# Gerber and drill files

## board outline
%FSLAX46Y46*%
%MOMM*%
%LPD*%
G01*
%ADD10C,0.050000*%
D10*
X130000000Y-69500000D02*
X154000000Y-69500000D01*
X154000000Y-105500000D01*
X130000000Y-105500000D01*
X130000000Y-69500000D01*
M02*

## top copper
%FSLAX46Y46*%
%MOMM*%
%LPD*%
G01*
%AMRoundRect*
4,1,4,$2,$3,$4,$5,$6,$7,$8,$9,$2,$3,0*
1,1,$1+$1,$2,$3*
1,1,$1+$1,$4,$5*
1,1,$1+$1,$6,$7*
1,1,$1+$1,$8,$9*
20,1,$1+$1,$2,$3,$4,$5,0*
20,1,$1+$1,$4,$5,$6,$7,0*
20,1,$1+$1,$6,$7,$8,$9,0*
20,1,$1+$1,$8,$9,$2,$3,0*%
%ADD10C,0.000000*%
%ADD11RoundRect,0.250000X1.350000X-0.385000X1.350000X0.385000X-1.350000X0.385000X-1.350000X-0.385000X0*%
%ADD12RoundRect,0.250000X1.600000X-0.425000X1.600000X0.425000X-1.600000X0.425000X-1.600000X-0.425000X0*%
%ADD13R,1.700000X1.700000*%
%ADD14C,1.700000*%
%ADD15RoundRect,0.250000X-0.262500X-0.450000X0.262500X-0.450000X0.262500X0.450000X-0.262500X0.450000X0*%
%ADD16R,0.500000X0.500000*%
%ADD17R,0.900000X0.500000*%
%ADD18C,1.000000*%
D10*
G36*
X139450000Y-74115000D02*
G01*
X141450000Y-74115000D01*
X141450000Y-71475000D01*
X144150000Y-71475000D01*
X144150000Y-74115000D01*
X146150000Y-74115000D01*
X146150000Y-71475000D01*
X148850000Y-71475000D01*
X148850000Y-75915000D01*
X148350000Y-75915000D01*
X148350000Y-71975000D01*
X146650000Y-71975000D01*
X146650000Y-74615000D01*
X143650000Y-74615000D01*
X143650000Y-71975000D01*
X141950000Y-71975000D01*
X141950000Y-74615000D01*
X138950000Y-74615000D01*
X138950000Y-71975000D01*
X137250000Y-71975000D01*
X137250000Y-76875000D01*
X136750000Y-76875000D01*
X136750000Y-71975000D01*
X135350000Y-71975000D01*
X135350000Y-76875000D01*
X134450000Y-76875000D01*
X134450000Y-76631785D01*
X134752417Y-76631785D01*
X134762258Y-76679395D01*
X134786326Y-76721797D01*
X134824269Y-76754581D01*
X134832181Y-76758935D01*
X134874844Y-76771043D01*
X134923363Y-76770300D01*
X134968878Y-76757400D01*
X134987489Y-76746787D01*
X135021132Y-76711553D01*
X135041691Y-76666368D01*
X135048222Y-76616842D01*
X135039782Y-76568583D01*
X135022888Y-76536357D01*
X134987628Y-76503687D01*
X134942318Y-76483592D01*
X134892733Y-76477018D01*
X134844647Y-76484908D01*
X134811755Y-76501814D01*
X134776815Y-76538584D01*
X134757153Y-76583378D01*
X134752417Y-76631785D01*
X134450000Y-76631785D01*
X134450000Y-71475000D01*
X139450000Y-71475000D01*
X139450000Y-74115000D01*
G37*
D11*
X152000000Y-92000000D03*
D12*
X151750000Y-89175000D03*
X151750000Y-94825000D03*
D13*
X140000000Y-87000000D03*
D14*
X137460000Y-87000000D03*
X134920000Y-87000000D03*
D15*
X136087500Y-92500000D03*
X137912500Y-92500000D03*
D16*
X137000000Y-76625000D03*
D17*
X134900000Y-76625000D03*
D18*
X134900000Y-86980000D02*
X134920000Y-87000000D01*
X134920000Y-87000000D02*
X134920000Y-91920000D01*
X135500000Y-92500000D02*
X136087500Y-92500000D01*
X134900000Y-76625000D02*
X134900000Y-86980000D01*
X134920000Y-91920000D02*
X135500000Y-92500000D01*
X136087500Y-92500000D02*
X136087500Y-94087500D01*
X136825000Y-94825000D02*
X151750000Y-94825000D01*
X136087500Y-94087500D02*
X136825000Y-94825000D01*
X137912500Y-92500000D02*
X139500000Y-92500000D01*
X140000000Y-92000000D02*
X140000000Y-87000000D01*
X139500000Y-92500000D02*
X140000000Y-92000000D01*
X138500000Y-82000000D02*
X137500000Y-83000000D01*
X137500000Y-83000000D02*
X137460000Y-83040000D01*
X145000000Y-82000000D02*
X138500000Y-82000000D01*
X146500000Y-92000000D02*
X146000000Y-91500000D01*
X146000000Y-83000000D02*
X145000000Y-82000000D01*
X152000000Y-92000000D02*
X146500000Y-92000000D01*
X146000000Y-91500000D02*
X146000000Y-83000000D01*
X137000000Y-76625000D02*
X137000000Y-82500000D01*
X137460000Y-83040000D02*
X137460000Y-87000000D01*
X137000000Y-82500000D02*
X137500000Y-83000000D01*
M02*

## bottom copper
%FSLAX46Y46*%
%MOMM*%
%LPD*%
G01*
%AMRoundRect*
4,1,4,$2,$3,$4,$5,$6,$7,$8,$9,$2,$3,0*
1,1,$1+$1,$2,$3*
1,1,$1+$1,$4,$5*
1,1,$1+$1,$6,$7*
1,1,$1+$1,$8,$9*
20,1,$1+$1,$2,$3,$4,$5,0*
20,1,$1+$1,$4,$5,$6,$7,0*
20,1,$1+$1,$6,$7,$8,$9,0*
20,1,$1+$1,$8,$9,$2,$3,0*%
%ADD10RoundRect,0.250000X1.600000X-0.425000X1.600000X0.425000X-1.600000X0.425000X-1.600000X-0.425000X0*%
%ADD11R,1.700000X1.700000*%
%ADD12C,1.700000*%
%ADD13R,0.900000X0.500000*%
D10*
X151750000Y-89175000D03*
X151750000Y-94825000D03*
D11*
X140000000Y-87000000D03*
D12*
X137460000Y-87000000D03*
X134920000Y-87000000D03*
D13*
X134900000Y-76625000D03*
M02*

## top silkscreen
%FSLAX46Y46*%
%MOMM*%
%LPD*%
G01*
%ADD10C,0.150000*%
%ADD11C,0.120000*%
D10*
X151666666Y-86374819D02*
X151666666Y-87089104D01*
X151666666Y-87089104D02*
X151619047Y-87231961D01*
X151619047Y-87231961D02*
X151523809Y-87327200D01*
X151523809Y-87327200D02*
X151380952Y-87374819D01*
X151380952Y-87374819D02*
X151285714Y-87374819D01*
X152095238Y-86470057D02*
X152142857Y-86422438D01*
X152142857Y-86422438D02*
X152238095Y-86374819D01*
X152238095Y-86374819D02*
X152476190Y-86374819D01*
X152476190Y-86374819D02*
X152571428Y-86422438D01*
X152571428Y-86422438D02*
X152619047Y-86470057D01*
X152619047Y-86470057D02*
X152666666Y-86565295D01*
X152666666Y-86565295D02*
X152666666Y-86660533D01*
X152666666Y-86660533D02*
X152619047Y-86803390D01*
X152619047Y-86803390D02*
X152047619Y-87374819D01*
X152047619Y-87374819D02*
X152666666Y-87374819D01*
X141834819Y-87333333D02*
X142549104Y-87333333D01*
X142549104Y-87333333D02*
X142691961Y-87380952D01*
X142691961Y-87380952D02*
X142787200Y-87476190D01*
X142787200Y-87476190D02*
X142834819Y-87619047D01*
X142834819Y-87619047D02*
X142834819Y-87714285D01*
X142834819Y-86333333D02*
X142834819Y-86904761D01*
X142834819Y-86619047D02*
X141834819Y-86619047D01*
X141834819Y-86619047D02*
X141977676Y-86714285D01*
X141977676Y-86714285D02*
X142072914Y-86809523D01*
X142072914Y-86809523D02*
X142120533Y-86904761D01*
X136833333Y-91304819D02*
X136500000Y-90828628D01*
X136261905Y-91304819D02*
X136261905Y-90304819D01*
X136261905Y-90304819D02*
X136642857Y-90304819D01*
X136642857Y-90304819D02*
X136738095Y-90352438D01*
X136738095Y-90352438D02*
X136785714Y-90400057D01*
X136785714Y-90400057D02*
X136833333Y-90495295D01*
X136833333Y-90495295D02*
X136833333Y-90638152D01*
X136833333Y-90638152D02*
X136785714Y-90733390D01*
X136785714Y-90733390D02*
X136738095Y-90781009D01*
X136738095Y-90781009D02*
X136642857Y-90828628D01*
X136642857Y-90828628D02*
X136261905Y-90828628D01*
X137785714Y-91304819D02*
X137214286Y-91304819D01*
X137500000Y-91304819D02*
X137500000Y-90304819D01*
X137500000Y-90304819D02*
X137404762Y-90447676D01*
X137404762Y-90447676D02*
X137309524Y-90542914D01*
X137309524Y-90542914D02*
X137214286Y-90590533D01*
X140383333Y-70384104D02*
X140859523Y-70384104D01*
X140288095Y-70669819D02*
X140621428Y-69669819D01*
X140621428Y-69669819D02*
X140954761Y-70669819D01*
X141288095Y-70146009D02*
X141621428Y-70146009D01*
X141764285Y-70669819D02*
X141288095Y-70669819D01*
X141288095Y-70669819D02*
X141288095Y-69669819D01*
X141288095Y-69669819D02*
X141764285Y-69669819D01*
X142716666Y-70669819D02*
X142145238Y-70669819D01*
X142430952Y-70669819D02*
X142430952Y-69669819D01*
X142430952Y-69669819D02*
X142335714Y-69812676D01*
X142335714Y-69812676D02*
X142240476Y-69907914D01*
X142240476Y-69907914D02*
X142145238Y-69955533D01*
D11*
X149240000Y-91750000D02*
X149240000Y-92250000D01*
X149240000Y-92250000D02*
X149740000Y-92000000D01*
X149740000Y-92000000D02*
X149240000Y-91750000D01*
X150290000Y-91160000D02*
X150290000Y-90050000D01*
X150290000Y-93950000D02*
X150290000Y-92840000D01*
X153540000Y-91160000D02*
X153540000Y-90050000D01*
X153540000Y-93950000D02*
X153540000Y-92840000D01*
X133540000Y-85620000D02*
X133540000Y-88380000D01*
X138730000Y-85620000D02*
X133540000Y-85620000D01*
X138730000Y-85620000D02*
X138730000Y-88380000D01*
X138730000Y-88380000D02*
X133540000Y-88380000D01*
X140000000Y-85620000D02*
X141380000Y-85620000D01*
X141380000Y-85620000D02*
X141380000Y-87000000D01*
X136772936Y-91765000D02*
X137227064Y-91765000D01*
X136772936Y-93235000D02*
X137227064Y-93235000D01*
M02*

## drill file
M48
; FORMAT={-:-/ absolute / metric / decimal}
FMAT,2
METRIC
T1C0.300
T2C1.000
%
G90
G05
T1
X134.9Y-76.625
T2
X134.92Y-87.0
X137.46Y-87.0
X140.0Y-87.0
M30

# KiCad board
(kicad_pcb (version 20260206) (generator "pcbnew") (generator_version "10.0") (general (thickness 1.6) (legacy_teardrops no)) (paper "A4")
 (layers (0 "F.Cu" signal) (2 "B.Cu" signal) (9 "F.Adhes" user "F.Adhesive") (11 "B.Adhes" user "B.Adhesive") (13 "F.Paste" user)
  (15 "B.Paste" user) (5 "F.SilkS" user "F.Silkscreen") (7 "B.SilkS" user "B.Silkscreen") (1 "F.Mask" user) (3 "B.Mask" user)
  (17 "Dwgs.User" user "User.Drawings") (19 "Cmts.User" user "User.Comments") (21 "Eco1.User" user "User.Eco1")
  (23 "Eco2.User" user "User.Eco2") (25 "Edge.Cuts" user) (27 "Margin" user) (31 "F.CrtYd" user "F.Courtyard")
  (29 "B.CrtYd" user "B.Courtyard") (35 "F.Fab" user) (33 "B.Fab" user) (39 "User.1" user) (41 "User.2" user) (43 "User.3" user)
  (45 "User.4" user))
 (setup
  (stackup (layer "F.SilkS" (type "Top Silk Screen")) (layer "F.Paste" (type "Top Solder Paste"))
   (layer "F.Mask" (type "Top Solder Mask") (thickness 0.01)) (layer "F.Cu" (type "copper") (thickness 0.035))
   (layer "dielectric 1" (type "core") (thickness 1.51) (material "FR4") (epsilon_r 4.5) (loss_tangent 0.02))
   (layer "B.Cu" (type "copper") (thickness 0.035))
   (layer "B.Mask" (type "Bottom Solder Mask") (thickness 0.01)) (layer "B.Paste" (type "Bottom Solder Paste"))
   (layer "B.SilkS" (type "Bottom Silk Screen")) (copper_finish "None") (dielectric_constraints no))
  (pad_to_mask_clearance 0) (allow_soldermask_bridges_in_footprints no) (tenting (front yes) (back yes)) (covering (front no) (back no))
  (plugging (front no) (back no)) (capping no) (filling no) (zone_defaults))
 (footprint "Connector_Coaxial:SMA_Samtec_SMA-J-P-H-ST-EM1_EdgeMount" (layer "F.Cu") (at 152 92)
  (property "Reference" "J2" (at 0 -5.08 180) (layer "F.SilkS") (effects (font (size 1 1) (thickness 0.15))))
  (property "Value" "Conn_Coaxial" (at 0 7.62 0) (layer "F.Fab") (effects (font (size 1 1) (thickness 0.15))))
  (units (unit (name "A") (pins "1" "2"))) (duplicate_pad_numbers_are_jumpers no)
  (fp_line (start -2.76 -0.25) (end -2.76 0.25) (stroke (width 0.12) (type solid)) (layer "F.SilkS"))
  (fp_line (start -2.76 0.25) (end -2.26 0) (stroke (width 0.12) (type solid)) (layer "F.SilkS"))
  (fp_line (start -2.26 0) (end -2.76 -0.25) (stroke (width 0.12) (type solid)) (layer "F.SilkS"))
  (fp_line (start -1.71 -0.84) (end -1.71 -1.95) (stroke (width 0.12) (type solid)) (layer "F.SilkS"))
  (fp_line (start -1.71 1.95) (end -1.71 0.84) (stroke (width 0.12) (type solid)) (layer "F.SilkS"))
  (fp_line (start 1.54 -0.84) (end 1.54 -1.95) (stroke (width 0.12) (type solid)) (layer "F.SilkS"))
  (fp_line (start 1.54 1.95) (end 1.54 0.84) (stroke (width 0.12) (type solid)) (layer "F.SilkS"))
  (pad "1" smd roundrect (at 0 0 90) (size 1.27 3.2) (layers "F.Cu" "F.Mask") (roundrect_rratio 0.1968503937) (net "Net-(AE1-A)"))
  (pad "2" smd roundrect (at -0.25 -2.825 90) (size 1.35 3.7) (layers "F.Cu" "F.Mask") (roundrect_rratio 0.1851851852) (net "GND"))
  (pad "2" smd roundrect (at -0.25 -2.825 90) (size 1.35 3.7) (layers "B.Cu" "B.Mask") (roundrect_rratio 0.1851851852) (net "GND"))
  (pad "2" smd roundrect (at -0.25 2.825 90) (size 1.35 3.7) (layers "F.Cu" "F.Mask") (roundrect_rratio 0.1851851852) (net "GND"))
  (pad "2" smd roundrect (at -0.25 2.825 90) (size 1.35 3.7) (layers "B.Cu" "B.Mask") (roundrect_rratio 0.1851851852) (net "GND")))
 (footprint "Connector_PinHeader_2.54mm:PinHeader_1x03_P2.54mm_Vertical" (layer "F.Cu") (at 140 87 -90)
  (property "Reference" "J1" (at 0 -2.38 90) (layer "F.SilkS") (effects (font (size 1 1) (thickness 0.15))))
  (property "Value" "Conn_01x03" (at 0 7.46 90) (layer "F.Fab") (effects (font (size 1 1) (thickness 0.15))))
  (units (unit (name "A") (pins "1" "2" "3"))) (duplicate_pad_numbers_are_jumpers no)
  (fp_line (start -1.38 6.46) (end 1.38 6.46) (stroke (width 0.12) (type solid)) (layer "F.SilkS"))
  (fp_line (start -1.38 1.27) (end -1.38 6.46) (stroke (width 0.12) (type solid)) (layer "F.SilkS"))
  (fp_line (start -1.38 1.27) (end 1.38 1.27) (stroke (width 0.12) (type solid)) (layer "F.SilkS"))
  (fp_line (start 1.38 1.27) (end 1.38 6.46) (stroke (width 0.12) (type solid)) (layer "F.SilkS"))
  (fp_line (start -1.38 0) (end -1.38 -1.38) (stroke (width 0.12) (type solid)) (layer "F.SilkS"))
  (fp_line (start -1.38 -1.38) (end 0 -1.38) (stroke (width 0.12) (type solid)) (layer "F.SilkS"))
  (pad "1" thru_hole rect (at 0 0 270) (size 1.7 1.7) (drill 1) (layers "*.Cu" "*.Mask") (remove_unused_layers no) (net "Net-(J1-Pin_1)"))
  (pad "2" thru_hole circle (at 0 2.54 270) (size 1.7 1.7) (drill 1) (layers "*.Cu" "*.Mask") (remove_unused_layers no) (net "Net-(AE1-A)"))
  (pad "3" thru_hole circle (at 0 5.08 270) (size 1.7 1.7) (drill 1) (layers "*.Cu" "*.Mask") (remove_unused_layers no) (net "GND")))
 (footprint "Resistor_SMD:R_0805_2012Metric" (layer "F.Cu") (at 137 92.5)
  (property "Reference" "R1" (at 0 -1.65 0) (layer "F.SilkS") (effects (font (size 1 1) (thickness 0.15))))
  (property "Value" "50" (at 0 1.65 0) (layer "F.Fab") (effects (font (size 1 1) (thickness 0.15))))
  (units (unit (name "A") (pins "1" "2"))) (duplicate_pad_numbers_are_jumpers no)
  (fp_line (start -0.227064 -0.735) (end 0.227064 -0.735) (stroke (width 0.12) (type solid)) (layer "F.SilkS"))
  (fp_line (start -0.227064 0.735) (end 0.227064 0.735) (stroke (width 0.12) (type solid)) (layer "F.SilkS"))
  (pad "1" smd roundrect (at -0.9125 0) (size 1.025 1.4) (layers "F.Cu" "F.Mask" "F.Paste") (roundrect_rratio 0.243902) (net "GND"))
  (pad "2" smd roundrect (at 0.9125 0) (size 1.025 1.4) (layers "F.Cu" "F.Mask" "F.Paste") (roundrect_rratio 0.243902)
   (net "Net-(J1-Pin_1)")))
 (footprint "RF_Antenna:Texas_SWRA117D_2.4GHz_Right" (layer "F.Cu") (at 137 76.625)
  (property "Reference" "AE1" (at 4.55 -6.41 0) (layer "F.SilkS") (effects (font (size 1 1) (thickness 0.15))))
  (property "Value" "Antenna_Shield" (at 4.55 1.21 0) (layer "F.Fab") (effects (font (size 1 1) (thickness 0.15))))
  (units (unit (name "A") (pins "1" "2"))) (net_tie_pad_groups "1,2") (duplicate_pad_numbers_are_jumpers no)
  (fp_poly
   (pts (xy 2.45 -2.51) (xy 4.45 -2.51) (xy 4.45 -5.15) (xy 7.15 -5.15) (xy 7.15 -2.51) (xy 9.15 -2.51) (xy 9.15 -5.15) (xy 11.85 -5.15)
    (xy 11.85 -0.71) (xy 11.35 -0.71) (xy 11.35 -4.65) (xy 9.65 -4.65) (xy 9.65 -2.01) (xy 6.65 -2.01) (xy 6.65 -4.65) (xy 4.95 -4.65)
    (xy 4.95 -2.01) (xy 1.95 -2.01) (xy 1.95 -4.65) (xy 0.25 -4.65) (xy 0.25 0.25) (xy -0.25 0.25) (xy -0.25 -4.65) (xy -1.65 -4.65)
    (xy -1.65 0.25) (xy -2.55 0.25) (xy -2.55 0.006785) (xy -2.247583 0.006785) (xy -2.237742 0.054395) (xy -2.213674 0.096797)
    (xy -2.175731 0.129581) (xy -2.167819 0.133935) (xy -2.125156 0.146043) (xy -2.076637 0.1453) (xy -2.031122 0.1324)
    (xy -2.012511 0.121787) (xy -1.978868 0.086553) (xy -1.958309 0.041368) (xy -1.951778 -0.008158) (xy -1.960218 -0.056417)
    (xy -1.977112 -0.088643) (xy -2.012372 -0.121313) (xy -2.057682 -0.141408) (xy -2.107267 -0.147982) (xy -2.155353 -0.140092)
    (xy -2.188245 -0.123186) (xy -2.223185 -0.086416) (xy -2.242847 -0.041622) (xy -2.247583 0.006785) (xy -2.55 0.006785) (xy -2.55 -5.15)
    (xy 2.45 -5.15) (xy 2.45 -2.51))
   (stroke (width 0) (type solid)) (fill yes) (layer "F.Cu"))
  (pad "1" connect rect (at 0 0) (size 0.5 0.5) (layers "F.Cu") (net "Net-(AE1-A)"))
  (pad "2" thru_hole rect (at -2.1 0) (size 0.9 0.5) (drill 0.3) (layers "*.Cu") (remove_unused_layers no) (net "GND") (zone_connect 2)))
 (gr_rect (start 130 69.5) (end 154 105.5) (stroke (width 0.05) (type default)) (fill no) (layer "Edge.Cuts"))
 (segment (start 134.9 86.98) (end 134.92 87) (width 1) (layer "F.Cu") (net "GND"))
 (segment (start 134.92 87) (end 134.92 91.92) (width 1) (layer "F.Cu") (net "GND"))
 (segment (start 135.5 92.5) (end 136.0875 92.5) (width 1) (layer "F.Cu") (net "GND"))
 (segment (start 134.9 76.625) (end 134.9 86.98) (width 1) (layer "F.Cu") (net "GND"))
 (segment (start 134.92 91.92) (end 135.5 92.5) (width 1) (layer "F.Cu") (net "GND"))
 (segment (start 136.0875 92.5) (end 136.0875 94.0875) (width 1) (layer "F.Cu") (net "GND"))
 (segment (start 136.825 94.825) (end 151.75 94.825) (width 1) (layer "F.Cu") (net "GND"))
 (segment (start 136.0875 94.0875) (end 136.825 94.825) (width 1) (layer "F.Cu") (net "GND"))
 (segment (start 137.9125 92.5) (end 139.5 92.5) (width 1) (layer "F.Cu") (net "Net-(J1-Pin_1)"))
 (segment (start 140 92) (end 140 87) (width 1) (layer "F.Cu") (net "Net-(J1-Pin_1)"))
 (segment (start 139.5 92.5) (end 140 92) (width 1) (layer "F.Cu") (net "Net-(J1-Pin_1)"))
 (segment (start 138.5 82) (end 137.5 83) (width 1) (layer "F.Cu") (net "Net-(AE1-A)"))
 (segment (start 137.5 83) (end 137.46 83.04) (width 1) (layer "F.Cu") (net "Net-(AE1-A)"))
 (segment (start 145 82) (end 138.5 82) (width 1) (layer "F.Cu") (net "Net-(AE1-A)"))
 (segment (start 146.5 92) (end 146 91.5) (width 1) (layer "F.Cu") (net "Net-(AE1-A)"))
 (segment (start 146 83) (end 145 82) (width 1) (layer "F.Cu") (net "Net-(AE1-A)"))
 (segment (start 152 92) (end 146.5 92) (width 1) (layer "F.Cu") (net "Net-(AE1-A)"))
 (segment (start 146 91.5) (end 146 83) (width 1) (layer "F.Cu") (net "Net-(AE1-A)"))
 (segment (start 137 76.625) (end 137 82.5) (width 1) (layer "F.Cu") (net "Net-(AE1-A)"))
 (segment (start 137.46 83.04) (end 137.46 87) (width 1) (layer "F.Cu") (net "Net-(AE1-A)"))
 (segment (start 137 82.5) (end 137.5 83) (width 1) (layer "F.Cu") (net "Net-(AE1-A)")))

